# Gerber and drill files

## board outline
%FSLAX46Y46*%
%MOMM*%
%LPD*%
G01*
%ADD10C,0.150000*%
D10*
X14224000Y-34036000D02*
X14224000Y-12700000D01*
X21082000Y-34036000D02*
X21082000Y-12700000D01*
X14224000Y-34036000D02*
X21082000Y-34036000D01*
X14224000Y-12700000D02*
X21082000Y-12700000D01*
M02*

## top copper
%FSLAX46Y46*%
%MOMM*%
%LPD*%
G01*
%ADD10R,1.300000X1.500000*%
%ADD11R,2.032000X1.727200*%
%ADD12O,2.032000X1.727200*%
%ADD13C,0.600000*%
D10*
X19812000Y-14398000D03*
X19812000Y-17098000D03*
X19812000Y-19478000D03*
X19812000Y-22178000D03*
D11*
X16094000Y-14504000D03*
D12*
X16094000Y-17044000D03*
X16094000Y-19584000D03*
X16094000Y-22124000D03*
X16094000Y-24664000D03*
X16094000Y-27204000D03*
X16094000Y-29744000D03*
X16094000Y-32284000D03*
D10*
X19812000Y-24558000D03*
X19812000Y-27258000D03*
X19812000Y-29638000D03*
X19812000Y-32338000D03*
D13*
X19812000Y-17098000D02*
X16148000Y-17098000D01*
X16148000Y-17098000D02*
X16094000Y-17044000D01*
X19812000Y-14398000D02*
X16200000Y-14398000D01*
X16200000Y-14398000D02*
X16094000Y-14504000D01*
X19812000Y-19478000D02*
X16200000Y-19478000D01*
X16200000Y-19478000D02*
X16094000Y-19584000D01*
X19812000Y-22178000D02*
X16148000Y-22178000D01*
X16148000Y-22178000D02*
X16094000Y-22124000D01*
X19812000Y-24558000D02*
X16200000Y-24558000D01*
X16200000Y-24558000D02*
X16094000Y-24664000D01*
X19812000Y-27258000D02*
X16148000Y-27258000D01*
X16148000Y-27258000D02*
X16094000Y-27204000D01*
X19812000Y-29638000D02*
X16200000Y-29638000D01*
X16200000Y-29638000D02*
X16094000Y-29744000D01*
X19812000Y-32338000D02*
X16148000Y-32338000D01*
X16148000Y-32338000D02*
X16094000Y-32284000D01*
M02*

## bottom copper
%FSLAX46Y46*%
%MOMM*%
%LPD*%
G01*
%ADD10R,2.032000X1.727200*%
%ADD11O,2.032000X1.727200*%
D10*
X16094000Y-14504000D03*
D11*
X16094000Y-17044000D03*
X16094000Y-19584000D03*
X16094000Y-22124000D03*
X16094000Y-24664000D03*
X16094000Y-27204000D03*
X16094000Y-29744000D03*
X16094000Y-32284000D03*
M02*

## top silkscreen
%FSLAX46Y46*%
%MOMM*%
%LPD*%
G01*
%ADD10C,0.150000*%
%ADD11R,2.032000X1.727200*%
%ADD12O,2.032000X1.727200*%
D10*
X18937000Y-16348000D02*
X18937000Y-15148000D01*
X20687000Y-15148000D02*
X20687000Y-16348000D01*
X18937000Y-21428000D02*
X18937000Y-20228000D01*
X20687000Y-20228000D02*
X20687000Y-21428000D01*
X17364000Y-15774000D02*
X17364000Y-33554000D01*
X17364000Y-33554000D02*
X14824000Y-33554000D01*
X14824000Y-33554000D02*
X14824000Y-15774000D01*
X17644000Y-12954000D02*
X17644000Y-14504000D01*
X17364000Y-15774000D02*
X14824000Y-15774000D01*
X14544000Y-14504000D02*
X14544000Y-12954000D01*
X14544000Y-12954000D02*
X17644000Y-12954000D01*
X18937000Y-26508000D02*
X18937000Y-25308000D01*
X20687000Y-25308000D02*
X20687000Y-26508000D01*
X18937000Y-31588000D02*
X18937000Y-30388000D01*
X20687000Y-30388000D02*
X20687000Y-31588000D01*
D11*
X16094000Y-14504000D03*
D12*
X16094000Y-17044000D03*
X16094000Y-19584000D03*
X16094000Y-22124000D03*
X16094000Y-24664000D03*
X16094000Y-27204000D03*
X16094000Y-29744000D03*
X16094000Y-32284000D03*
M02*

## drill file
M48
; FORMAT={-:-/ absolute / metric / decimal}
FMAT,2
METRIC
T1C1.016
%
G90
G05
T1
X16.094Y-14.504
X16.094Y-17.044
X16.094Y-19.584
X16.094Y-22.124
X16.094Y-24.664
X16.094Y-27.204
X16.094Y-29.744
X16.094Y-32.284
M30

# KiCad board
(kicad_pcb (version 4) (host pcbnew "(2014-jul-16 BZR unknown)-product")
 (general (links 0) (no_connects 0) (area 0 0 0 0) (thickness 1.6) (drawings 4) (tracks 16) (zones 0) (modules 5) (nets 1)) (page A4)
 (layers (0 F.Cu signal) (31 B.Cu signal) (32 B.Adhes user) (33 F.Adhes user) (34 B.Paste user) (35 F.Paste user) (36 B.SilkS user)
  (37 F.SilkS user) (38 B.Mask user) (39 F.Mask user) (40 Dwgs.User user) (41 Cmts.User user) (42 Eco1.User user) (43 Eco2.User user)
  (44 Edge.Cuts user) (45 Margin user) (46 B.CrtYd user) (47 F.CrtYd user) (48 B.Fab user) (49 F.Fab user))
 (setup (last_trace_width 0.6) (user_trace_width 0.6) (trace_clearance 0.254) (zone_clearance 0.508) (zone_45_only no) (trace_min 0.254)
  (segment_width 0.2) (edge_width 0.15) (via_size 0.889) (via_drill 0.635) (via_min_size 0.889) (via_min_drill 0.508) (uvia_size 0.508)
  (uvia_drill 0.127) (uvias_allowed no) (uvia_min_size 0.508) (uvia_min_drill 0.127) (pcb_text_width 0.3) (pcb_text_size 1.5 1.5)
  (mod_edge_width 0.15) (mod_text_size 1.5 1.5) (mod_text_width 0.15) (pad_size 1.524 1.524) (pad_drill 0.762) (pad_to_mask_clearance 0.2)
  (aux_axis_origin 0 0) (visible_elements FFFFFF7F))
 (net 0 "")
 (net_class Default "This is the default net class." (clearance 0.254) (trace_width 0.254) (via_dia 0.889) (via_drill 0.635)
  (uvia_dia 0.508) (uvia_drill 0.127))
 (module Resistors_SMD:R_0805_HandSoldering (layer F.Cu) (at 19.812 15.748 270)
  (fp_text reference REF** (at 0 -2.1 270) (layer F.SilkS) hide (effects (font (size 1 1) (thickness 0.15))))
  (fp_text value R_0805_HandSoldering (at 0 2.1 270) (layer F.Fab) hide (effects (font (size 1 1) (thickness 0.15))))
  (fp_line (start 0.6 0.875) (end -0.6 0.875) (layer F.SilkS) (width 0.15))
  (fp_line (start -0.6 -0.875) (end 0.6 -0.875) (layer F.SilkS) (width 0.15))
  (pad 1 smd rect (at -1.35 0 270) (size 1.5 1.3) (layers F.Cu F.Paste F.Mask))
  (pad 2 smd rect (at 1.35 0 270) (size 1.5 1.3) (layers F.Cu F.Paste F.Mask)))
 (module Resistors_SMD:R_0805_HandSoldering (layer F.Cu) (at 19.812 20.828 270)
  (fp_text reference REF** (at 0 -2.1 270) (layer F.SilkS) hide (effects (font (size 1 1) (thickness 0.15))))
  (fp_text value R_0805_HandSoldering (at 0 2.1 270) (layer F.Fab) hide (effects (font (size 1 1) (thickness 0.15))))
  (fp_line (start 0.6 0.875) (end -0.6 0.875) (layer F.SilkS) (width 0.15))
  (fp_line (start -0.6 -0.875) (end 0.6 -0.875) (layer F.SilkS) (width 0.15))
  (pad 1 smd rect (at -1.35 0 270) (size 1.5 1.3) (layers F.Cu F.Paste F.Mask))
  (pad 2 smd rect (at 1.35 0 270) (size 1.5 1.3) (layers F.Cu F.Paste F.Mask)))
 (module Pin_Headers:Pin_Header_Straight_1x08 (layer F.Cu) (at 16.094 14.504)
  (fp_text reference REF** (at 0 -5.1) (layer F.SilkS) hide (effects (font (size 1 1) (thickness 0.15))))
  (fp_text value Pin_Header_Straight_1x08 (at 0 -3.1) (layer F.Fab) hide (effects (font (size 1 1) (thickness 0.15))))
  (fp_line (start 1.27 1.27) (end 1.27 19.05) (layer F.SilkS) (width 0.15))
  (fp_line (start 1.27 19.05) (end -1.27 19.05) (layer F.SilkS) (width 0.15))
  (fp_line (start -1.27 19.05) (end -1.27 1.27) (layer F.SilkS) (width 0.15))
  (fp_line (start 1.55 -1.55) (end 1.55 0) (layer F.SilkS) (width 0.15))
  (fp_line (start 1.27 1.27) (end -1.27 1.27) (layer F.SilkS) (width 0.15))
  (fp_line (start -1.55 0) (end -1.55 -1.55) (layer F.SilkS) (width 0.15))
  (fp_line (start -1.55 -1.55) (end 1.55 -1.55) (layer F.SilkS) (width 0.15))
  (pad 1 thru_hole rect (at 0 0) (size 2.032 1.7272) (drill 1.016) (layers *.Cu *.Mask F.SilkS))
  (pad 2 thru_hole oval (at 0 2.54) (size 2.032 1.7272) (drill 1.016) (layers *.Cu *.Mask F.SilkS))
  (pad 3 thru_hole oval (at 0 5.08) (size 2.032 1.7272) (drill 1.016) (layers *.Cu *.Mask F.SilkS))
  (pad 4 thru_hole oval (at 0 7.62) (size 2.032 1.7272) (drill 1.016) (layers *.Cu *.Mask F.SilkS))
  (pad 5 thru_hole oval (at 0 10.16) (size 2.032 1.7272) (drill 1.016) (layers *.Cu *.Mask F.SilkS))
  (pad 6 thru_hole oval (at 0 12.7) (size 2.032 1.7272) (drill 1.016) (layers *.Cu *.Mask F.SilkS))
  (pad 7 thru_hole oval (at 0 15.24) (size 2.032 1.7272) (drill 1.016) (layers *.Cu *.Mask F.SilkS))
  (pad 8 thru_hole oval (at 0 17.78) (size 2.032 1.7272) (drill 1.016) (layers *.Cu *.Mask F.SilkS)))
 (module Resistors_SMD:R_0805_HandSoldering (layer F.Cu) (at 19.812 25.908 270)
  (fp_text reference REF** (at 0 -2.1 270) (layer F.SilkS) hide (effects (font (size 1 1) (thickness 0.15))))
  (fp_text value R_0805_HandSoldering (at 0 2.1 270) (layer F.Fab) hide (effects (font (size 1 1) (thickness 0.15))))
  (fp_line (start 0.6 0.875) (end -0.6 0.875) (layer F.SilkS) (width 0.15))
  (fp_line (start -0.6 -0.875) (end 0.6 -0.875) (layer F.SilkS) (width 0.15))
  (pad 1 smd rect (at -1.35 0 270) (size 1.5 1.3) (layers F.Cu F.Paste F.Mask))
  (pad 2 smd rect (at 1.35 0 270) (size 1.5 1.3) (layers F.Cu F.Paste F.Mask)))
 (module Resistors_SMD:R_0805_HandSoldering (layer F.Cu) (at 19.812 30.988 270)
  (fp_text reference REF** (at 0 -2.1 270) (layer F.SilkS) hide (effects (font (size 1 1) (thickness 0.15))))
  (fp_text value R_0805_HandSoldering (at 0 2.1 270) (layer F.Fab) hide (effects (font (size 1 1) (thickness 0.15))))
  (fp_line (start 0.6 0.875) (end -0.6 0.875) (layer F.SilkS) (width 0.15))
  (fp_line (start -0.6 -0.875) (end 0.6 -0.875) (layer F.SilkS) (width 0.15))
  (pad 1 smd rect (at -1.35 0 270) (size 1.5 1.3) (layers F.Cu F.Paste F.Mask))
  (pad 2 smd rect (at 1.35 0 270) (size 1.5 1.3) (layers F.Cu F.Paste F.Mask)))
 (gr_line (start 14.224 34.036) (end 14.224 12.7) (angle 90) (layer Edge.Cuts) (width 0.15))
 (gr_line (start 21.082 34.036) (end 21.082 12.7) (angle 90) (layer Edge.Cuts) (width 0.15))
 (gr_line (start 14.224 34.036) (end 21.082 34.036) (angle 90) (layer Edge.Cuts) (width 0.15))
 (gr_line (start 14.224 12.7) (end 21.082 12.7) (angle 90) (layer Edge.Cuts) (width 0.15))
 (segment (start 19.812 17.098) (end 16.148 17.098) (width 0.6) (layer F.Cu) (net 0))
 (segment (start 16.148 17.098) (end 16.094 17.044) (width 0.6) (layer F.Cu) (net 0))
 (segment (start 19.812 14.398) (end 16.2 14.398) (width 0.6) (layer F.Cu) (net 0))
 (segment (start 16.2 14.398) (end 16.094 14.504) (width 0.6) (layer F.Cu) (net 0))
 (segment (start 19.812 19.478) (end 16.2 19.478) (width 0.6) (layer F.Cu) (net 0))
 (segment (start 16.2 19.478) (end 16.094 19.584) (width 0.6) (layer F.Cu) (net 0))
 (segment (start 19.812 22.178) (end 16.148 22.178) (width 0.6) (layer F.Cu) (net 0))
 (segment (start 16.148 22.178) (end 16.094 22.124) (width 0.6) (layer F.Cu) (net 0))
 (segment (start 19.812 24.558) (end 16.2 24.558) (width 0.6) (layer F.Cu) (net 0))
 (segment (start 16.2 24.558) (end 16.094 24.664) (width 0.6) (layer F.Cu) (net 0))
 (segment (start 19.812 27.258) (end 16.148 27.258) (width 0.6) (layer F.Cu) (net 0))
 (segment (start 16.148 27.258) (end 16.094 27.204) (width 0.6) (layer F.Cu) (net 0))
 (segment (start 19.812 29.638) (end 16.2 29.638) (width 0.6) (layer F.Cu) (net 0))
 (segment (start 16.2 29.638) (end 16.094 29.744) (width 0.6) (layer F.Cu) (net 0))
 (segment (start 19.812 32.338) (end 16.148 32.338) (width 0.6) (layer F.Cu) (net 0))
 (segment (start 16.148 32.338) (end 16.094 32.284) (width 0.6) (layer F.Cu) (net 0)))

